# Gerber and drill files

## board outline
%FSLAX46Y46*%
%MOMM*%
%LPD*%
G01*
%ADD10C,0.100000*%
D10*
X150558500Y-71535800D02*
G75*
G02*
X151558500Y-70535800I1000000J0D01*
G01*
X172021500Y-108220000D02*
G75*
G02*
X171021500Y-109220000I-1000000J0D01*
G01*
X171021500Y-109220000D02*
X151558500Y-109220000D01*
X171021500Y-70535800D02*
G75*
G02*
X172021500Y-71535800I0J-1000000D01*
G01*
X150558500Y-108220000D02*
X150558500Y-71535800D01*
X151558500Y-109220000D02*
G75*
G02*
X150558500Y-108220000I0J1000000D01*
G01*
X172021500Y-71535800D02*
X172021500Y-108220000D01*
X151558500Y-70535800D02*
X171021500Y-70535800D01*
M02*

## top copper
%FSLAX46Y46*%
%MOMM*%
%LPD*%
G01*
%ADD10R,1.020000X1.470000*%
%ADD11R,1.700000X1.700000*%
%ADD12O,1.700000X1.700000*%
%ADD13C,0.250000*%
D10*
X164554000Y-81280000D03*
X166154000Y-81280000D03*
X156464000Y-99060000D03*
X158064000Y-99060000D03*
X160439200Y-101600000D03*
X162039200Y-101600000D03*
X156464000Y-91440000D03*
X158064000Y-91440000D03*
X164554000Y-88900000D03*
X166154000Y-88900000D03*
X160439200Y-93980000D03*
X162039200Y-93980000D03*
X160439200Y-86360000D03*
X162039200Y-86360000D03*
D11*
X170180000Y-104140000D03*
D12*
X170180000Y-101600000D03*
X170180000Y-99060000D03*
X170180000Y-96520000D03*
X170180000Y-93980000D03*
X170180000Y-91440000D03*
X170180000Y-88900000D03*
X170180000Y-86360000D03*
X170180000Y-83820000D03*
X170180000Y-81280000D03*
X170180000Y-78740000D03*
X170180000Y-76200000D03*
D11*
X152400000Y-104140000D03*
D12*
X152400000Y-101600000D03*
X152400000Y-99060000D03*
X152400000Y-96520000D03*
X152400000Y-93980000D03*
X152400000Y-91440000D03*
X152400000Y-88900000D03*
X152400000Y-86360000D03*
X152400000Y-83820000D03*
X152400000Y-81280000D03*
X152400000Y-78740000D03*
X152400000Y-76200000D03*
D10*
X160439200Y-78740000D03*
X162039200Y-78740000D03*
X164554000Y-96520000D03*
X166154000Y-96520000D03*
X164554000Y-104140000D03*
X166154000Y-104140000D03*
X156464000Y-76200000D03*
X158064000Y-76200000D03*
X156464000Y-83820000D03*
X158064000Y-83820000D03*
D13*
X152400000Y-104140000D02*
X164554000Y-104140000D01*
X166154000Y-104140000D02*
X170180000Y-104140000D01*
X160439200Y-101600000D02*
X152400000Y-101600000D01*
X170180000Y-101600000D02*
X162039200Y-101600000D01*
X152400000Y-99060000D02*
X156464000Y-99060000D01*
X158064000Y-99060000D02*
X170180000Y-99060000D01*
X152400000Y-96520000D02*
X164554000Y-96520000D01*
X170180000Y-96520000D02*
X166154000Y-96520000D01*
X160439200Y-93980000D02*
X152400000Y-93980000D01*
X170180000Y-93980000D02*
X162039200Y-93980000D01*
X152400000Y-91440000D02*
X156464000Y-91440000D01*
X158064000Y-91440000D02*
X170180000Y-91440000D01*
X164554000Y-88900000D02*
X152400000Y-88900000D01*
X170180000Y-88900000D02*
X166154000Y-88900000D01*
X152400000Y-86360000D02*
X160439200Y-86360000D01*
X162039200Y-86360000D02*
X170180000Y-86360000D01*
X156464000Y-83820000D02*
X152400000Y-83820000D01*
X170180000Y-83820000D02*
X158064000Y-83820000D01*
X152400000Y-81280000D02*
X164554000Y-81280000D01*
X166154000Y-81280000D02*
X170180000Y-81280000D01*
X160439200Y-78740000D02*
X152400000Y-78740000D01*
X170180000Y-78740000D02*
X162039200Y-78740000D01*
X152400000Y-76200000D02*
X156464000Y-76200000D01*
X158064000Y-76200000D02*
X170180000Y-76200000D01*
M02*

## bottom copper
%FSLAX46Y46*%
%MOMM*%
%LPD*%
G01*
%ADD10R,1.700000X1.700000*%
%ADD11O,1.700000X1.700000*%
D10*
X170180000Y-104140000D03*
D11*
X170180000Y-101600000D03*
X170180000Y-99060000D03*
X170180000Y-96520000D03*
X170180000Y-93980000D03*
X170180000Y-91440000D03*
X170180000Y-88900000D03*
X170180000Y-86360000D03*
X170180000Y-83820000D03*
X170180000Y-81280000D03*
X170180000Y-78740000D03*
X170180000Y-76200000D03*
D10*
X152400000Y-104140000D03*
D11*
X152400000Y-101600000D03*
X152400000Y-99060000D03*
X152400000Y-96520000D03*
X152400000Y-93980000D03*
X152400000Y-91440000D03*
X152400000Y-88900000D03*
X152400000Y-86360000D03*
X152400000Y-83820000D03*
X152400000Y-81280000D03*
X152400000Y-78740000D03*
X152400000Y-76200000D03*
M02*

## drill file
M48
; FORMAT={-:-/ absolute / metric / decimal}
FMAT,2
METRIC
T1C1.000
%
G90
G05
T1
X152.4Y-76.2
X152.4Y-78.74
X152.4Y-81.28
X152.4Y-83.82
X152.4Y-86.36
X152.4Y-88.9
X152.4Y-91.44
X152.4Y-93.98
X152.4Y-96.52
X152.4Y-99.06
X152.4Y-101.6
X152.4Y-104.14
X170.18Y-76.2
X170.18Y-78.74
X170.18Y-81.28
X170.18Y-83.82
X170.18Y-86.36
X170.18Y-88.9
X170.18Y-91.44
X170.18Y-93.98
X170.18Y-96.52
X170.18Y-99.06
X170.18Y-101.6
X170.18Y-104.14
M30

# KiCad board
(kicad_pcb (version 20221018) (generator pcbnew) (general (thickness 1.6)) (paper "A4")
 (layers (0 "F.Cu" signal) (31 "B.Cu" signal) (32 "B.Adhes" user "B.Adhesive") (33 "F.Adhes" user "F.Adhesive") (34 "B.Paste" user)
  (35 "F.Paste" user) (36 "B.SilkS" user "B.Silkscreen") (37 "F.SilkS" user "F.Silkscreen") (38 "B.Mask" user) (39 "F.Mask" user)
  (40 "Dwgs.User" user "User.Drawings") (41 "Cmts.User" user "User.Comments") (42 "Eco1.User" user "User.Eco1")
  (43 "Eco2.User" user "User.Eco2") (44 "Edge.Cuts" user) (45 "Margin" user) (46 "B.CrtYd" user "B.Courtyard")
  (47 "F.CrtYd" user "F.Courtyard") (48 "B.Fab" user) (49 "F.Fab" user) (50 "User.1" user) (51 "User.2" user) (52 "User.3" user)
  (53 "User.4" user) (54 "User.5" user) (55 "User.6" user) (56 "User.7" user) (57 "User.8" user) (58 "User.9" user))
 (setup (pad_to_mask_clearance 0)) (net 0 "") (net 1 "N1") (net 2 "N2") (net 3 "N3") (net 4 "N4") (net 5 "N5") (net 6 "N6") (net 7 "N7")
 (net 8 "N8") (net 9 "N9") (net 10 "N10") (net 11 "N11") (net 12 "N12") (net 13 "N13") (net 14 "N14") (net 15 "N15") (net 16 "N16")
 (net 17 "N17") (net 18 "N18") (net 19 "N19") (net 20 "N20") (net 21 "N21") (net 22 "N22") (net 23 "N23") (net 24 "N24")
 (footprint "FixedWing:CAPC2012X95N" (layer "F.Cu") (at 165.354 81.28)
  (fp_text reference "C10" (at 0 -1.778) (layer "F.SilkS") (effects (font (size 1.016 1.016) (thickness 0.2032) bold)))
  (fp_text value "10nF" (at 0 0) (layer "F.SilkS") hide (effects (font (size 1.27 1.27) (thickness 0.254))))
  (pad "1" smd rect (at -0.8 0) (size 1.02 1.47) (layers "F.Cu" "F.Paste" "F.Mask") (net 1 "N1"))
  (pad "2" smd rect (at 0.8 0) (size 1.02 1.47) (layers "F.Cu" "F.Paste" "F.Mask") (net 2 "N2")))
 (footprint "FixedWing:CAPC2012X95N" (layer "F.Cu") (at 157.264 99.06)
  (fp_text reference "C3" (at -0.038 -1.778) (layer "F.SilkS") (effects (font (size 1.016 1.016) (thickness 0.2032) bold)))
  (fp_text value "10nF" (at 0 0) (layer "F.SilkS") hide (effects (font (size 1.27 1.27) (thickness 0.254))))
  (pad "1" smd rect (at -0.8 0) (size 1.02 1.47) (layers "F.Cu" "F.Paste" "F.Mask") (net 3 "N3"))
  (pad "2" smd rect (at 0.8 0) (size 1.02 1.47) (layers "F.Cu" "F.Paste" "F.Mask") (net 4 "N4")))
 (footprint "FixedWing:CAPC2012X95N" (layer "F.Cu") (at 161.2392 101.6)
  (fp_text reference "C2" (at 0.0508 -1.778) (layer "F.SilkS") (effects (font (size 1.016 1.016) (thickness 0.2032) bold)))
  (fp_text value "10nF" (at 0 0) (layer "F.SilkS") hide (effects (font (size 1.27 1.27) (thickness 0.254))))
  (pad "1" smd rect (at -0.8 0) (size 1.02 1.47) (layers "F.Cu" "F.Paste" "F.Mask") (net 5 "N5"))
  (pad "2" smd rect (at 0.8 0) (size 1.02 1.47) (layers "F.Cu" "F.Paste" "F.Mask") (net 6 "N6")))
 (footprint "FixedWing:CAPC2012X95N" (layer "F.Cu") (at 157.264 91.44)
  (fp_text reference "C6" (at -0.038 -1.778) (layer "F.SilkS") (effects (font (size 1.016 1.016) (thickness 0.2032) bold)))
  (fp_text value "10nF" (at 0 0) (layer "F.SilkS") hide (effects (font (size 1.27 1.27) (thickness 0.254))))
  (pad "1" smd rect (at -0.8 0) (size 1.02 1.47) (layers "F.Cu" "F.Paste" "F.Mask") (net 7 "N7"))
  (pad "2" smd rect (at 0.8 0) (size 1.02 1.47) (layers "F.Cu" "F.Paste" "F.Mask") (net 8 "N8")))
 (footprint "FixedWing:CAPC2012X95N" (layer "F.Cu") (at 165.354 88.9)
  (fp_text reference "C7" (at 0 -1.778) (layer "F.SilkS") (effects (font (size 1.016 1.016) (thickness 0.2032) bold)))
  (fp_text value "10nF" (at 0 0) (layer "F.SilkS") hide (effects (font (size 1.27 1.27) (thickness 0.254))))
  (pad "1" smd rect (at -0.8 0) (size 1.02 1.47) (layers "F.Cu" "F.Paste" "F.Mask") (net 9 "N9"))
  (pad "2" smd rect (at 0.8 0) (size 1.02 1.47) (layers "F.Cu" "F.Paste" "F.Mask") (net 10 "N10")))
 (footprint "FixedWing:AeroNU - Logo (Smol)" (layer "F.Cu") (at 157.342549 108.843988)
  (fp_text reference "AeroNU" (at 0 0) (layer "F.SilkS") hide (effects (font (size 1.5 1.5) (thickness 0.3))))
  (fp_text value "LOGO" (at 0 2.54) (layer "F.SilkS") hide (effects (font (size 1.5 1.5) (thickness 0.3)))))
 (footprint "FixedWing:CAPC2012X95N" (layer "F.Cu") (at 161.2392 93.98)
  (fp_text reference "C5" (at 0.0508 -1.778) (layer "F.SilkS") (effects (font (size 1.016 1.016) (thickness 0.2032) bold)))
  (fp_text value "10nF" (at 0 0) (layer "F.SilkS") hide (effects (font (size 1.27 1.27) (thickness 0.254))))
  (pad "1" smd rect (at -0.8 0) (size 1.02 1.47) (layers "F.Cu" "F.Paste" "F.Mask") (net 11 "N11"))
  (pad "2" smd rect (at 0.8 0) (size 1.02 1.47) (layers "F.Cu" "F.Paste" "F.Mask") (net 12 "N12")))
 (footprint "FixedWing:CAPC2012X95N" (layer "F.Cu") (at 161.2392 86.36)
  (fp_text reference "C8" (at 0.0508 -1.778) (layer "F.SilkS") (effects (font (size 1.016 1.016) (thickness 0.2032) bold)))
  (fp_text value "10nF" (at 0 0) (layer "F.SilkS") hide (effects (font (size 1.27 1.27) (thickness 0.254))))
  (pad "1" smd rect (at -0.8 0) (size 1.02 1.47) (layers "F.Cu" "F.Paste" "F.Mask") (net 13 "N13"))
  (pad "2" smd rect (at 0.8 0) (size 1.02 1.47) (layers "F.Cu" "F.Paste" "F.Mask") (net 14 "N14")))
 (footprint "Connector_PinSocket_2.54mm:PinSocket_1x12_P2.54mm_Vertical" (layer "F.Cu") (at 170.18 104.14 180)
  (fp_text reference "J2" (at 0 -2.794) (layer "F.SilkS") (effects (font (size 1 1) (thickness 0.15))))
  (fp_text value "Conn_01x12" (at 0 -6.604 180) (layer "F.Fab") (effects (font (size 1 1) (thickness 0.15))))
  (pad "1" thru_hole rect (at 0 0 180) (size 1.7 1.7) (drill 1) (layers "*.Cu" "*.Mask") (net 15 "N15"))
  (pad "2" thru_hole oval (at 0 2.54 180) (size 1.7 1.7) (drill 1) (layers "*.Cu" "*.Mask") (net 6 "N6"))
  (pad "3" thru_hole oval (at 0 5.08 180) (size 1.7 1.7) (drill 1) (layers "*.Cu" "*.Mask") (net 4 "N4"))
  (pad "4" thru_hole oval (at 0 7.62 180) (size 1.7 1.7) (drill 1) (layers "*.Cu" "*.Mask") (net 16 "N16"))
  (pad "5" thru_hole oval (at 0 10.16 180) (size 1.7 1.7) (drill 1) (layers "*.Cu" "*.Mask") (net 12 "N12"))
  (pad "6" thru_hole oval (at 0 12.7 180) (size 1.7 1.7) (drill 1) (layers "*.Cu" "*.Mask") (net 8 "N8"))
  (pad "7" thru_hole oval (at 0 15.24 180) (size 1.7 1.7) (drill 1) (layers "*.Cu" "*.Mask") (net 10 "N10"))
  (pad "8" thru_hole oval (at 0 17.78 180) (size 1.7 1.7) (drill 1) (layers "*.Cu" "*.Mask") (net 14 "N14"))
  (pad "9" thru_hole oval (at 0 20.32 180) (size 1.7 1.7) (drill 1) (layers "*.Cu" "*.Mask") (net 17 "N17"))
  (pad "10" thru_hole oval (at 0 22.86 180) (size 1.7 1.7) (drill 1) (layers "*.Cu" "*.Mask") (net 2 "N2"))
  (pad "11" thru_hole oval (at 0 25.4 180) (size 1.7 1.7) (drill 1) (layers "*.Cu" "*.Mask") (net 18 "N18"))
  (pad "12" thru_hole oval (at 0 27.94 180) (size 1.7 1.7) (drill 1) (layers "*.Cu" "*.Mask") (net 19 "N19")))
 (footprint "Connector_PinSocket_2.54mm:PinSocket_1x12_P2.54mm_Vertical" (layer "F.Cu") (at 152.4 104.14 180)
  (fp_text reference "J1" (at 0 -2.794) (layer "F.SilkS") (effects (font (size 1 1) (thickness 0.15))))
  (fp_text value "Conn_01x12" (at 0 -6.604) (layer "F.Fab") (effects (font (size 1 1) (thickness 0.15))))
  (pad "1" thru_hole rect (at 0 0 180) (size 1.7 1.7) (drill 1) (layers "*.Cu" "*.Mask") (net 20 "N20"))
  (pad "2" thru_hole oval (at 0 2.54 180) (size 1.7 1.7) (drill 1) (layers "*.Cu" "*.Mask") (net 5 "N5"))
  (pad "3" thru_hole oval (at 0 5.08 180) (size 1.7 1.7) (drill 1) (layers "*.Cu" "*.Mask") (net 3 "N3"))
  (pad "4" thru_hole oval (at 0 7.62 180) (size 1.7 1.7) (drill 1) (layers "*.Cu" "*.Mask") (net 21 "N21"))
  (pad "5" thru_hole oval (at 0 10.16 180) (size 1.7 1.7) (drill 1) (layers "*.Cu" "*.Mask") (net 11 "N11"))
  (pad "6" thru_hole oval (at 0 12.7 180) (size 1.7 1.7) (drill 1) (layers "*.Cu" "*.Mask") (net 7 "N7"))
  (pad "7" thru_hole oval (at 0 15.24 180) (size 1.7 1.7) (drill 1) (layers "*.Cu" "*.Mask") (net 9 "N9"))
  (pad "8" thru_hole oval (at 0 17.78 180) (size 1.7 1.7) (drill 1) (layers "*.Cu" "*.Mask") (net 13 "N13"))
  (pad "9" thru_hole oval (at 0 20.32 180) (size 1.7 1.7) (drill 1) (layers "*.Cu" "*.Mask") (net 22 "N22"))
  (pad "10" thru_hole oval (at 0 22.86 180) (size 1.7 1.7) (drill 1) (layers "*.Cu" "*.Mask") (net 1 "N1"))
  (pad "11" thru_hole oval (at 0 25.4 180) (size 1.7 1.7) (drill 1) (layers "*.Cu" "*.Mask") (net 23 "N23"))
  (pad "12" thru_hole oval (at 0 27.94 180) (size 1.7 1.7) (drill 1) (layers "*.Cu" "*.Mask") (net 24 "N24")))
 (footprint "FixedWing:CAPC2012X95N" (layer "F.Cu") (at 161.2392 78.74)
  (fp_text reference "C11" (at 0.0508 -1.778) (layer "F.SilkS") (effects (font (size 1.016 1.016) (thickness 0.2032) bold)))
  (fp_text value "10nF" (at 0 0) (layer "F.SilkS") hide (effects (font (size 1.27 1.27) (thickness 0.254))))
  (pad "1" smd rect (at -0.8 0) (size 1.02 1.47) (layers "F.Cu" "F.Paste" "F.Mask") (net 23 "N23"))
  (pad "2" smd rect (at 0.8 0) (size 1.02 1.47) (layers "F.Cu" "F.Paste" "F.Mask") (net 18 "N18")))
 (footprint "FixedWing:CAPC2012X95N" (layer "F.Cu") (at 165.354 96.52)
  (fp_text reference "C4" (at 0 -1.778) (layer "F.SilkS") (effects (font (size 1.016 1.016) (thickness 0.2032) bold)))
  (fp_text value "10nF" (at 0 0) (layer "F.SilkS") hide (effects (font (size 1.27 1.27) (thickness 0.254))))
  (pad "1" smd rect (at -0.8 0) (size 1.02 1.47) (layers "F.Cu" "F.Paste" "F.Mask") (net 21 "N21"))
  (pad "2" smd rect (at 0.8 0) (size 1.02 1.47) (layers "F.Cu" "F.Paste" "F.Mask") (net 16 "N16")))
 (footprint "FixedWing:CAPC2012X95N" (layer "F.Cu") (at 165.354 104.14)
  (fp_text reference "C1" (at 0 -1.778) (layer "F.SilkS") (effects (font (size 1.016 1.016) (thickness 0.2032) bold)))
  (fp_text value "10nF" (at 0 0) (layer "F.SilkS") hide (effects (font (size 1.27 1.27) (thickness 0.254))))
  (pad "1" smd rect (at -0.8 0) (size 1.02 1.47) (layers "F.Cu" "F.Paste" "F.Mask") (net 20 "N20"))
  (pad "2" smd rect (at 0.8 0) (size 1.02 1.47) (layers "F.Cu" "F.Paste" "F.Mask") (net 15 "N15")))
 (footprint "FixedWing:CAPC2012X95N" (layer "F.Cu") (at 157.264 76.2)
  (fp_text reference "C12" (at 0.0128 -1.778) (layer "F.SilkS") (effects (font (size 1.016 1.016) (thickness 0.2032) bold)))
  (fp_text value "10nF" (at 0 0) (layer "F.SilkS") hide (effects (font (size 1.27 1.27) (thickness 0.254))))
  (pad "1" smd rect (at -0.8 0) (size 1.02 1.47) (layers "F.Cu" "F.Paste" "F.Mask") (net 24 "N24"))
  (pad "2" smd rect (at 0.8 0) (size 1.02 1.47) (layers "F.Cu" "F.Paste" "F.Mask") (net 19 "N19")))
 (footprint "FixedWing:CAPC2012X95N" (layer "F.Cu") (at 157.264 83.82)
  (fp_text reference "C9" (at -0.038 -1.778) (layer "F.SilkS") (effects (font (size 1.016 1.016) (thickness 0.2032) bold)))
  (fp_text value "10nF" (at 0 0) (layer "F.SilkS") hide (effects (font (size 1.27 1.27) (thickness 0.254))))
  (pad "1" smd rect (at -0.8 0) (size 1.02 1.47) (layers "F.Cu" "F.Paste" "F.Mask") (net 22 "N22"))
  (pad "2" smd rect (at 0.8 0) (size 1.02 1.47) (layers "F.Cu" "F.Paste" "F.Mask") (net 17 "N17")))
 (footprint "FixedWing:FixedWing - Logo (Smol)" (layer "F.Cu") (at 165.354 72.644)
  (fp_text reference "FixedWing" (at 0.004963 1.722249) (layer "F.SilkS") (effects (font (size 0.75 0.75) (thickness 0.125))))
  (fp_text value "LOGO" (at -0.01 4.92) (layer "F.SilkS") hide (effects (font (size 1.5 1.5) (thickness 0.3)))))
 (gr_arc (start 150.5585 71.5358) (mid 150.851393 70.828693) (end 151.5585 70.5358) (stroke (width 0.1) (type default)) (layer "Edge.Cuts"))
 (gr_arc (start 172.0215 108.22) (mid 171.728607 108.927107) (end 171.0215 109.22) (stroke (width 0.1) (type default)) (layer "Edge.Cuts"))
 (gr_line (start 171.0215 109.22) (end 151.5585 109.22) (stroke (width 0.1) (type default)) (layer "Edge.Cuts"))
 (gr_arc (start 171.0215 70.5358) (mid 171.728607 70.828693) (end 172.0215 71.5358) (stroke (width 0.1) (type default)) (layer "Edge.Cuts"))
 (gr_line (start 150.5585 108.22) (end 150.5585 71.5358) (stroke (width 0.1) (type default)) (layer "Edge.Cuts"))
 (gr_arc (start 151.5585 109.22) (mid 150.851393 108.927107) (end 150.5585 108.22) (stroke (width 0.1) (type default)) (layer "Edge.Cuts"))
 (gr_line (start 172.0215 71.5358) (end 172.0215 108.22) (stroke (width 0.1) (type default)) (layer "Edge.Cuts"))
 (gr_line (start 151.5585 70.5358) (end 171.0215 70.5358) (stroke (width 0.1) (type default)) (layer "Edge.Cuts"))
 (segment (start 152.4 104.14) (end 164.554 104.14) (width 0.25) (layer "F.Cu") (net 20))
 (segment (start 166.154 104.14) (end 170.18 104.14) (width 0.25) (layer "F.Cu") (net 15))
 (segment (start 160.4392 101.6) (end 152.4 101.6) (width 0.25) (layer "F.Cu") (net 5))
 (segment (start 170.18 101.6) (end 162.0392 101.6) (width 0.25) (layer "F.Cu") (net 6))
 (segment (start 152.4 99.06) (end 156.464 99.06) (width 0.25) (layer "F.Cu") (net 3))
 (segment (start 158.064 99.06) (end 170.18 99.06) (width 0.25) (layer "F.Cu") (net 4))
 (segment (start 152.4 96.52) (end 164.554 96.52) (width 0.25) (layer "F.Cu") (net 21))
 (segment (start 170.18 96.52) (end 166.154 96.52) (width 0.25) (layer "F.Cu") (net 16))
 (segment (start 160.4392 93.98) (end 152.4 93.98) (width 0.25) (layer "F.Cu") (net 11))
 (segment (start 170.18 93.98) (end 162.0392 93.98) (width 0.25) (layer "F.Cu") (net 12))
 (segment (start 152.4 91.44) (end 156.464 91.44) (width 0.25) (layer "F.Cu") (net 7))
 (segment (start 158.064 91.44) (end 170.18 91.44) (width 0.25) (layer "F.Cu") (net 8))
 (segment (start 164.554 88.9) (end 152.4 88.9) (width 0.25) (layer "F.Cu") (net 9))
 (segment (start 170.18 88.9) (end 166.154 88.9) (width 0.25) (layer "F.Cu") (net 10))
 (segment (start 152.4 86.36) (end 160.4392 86.36) (width 0.25) (layer "F.Cu") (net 13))
 (segment (start 162.0392 86.36) (end 170.18 86.36) (width 0.25) (layer "F.Cu") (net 14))
 (segment (start 156.464 83.82) (end 152.4 83.82) (width 0.25) (layer "F.Cu") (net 22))
 (segment (start 170.18 83.82) (end 158.064 83.82) (width 0.25) (layer "F.Cu") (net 17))
 (segment (start 152.4 81.28) (end 164.554 81.28) (width 0.25) (layer "F.Cu") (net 1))
 (segment (start 166.154 81.28) (end 170.18 81.28) (width 0.25) (layer "F.Cu") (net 2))
 (segment (start 160.4392 78.74) (end 152.4 78.74) (width 0.25) (layer "F.Cu") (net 23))
 (segment (start 170.18 78.74) (end 162.0392 78.74) (width 0.25) (layer "F.Cu") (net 18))
 (segment (start 152.4 76.2) (end 156.464 76.2) (width 0.25) (layer "F.Cu") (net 24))
 (segment (start 158.064 76.2) (end 170.18 76.2) (width 0.25) (layer "F.Cu") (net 19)))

